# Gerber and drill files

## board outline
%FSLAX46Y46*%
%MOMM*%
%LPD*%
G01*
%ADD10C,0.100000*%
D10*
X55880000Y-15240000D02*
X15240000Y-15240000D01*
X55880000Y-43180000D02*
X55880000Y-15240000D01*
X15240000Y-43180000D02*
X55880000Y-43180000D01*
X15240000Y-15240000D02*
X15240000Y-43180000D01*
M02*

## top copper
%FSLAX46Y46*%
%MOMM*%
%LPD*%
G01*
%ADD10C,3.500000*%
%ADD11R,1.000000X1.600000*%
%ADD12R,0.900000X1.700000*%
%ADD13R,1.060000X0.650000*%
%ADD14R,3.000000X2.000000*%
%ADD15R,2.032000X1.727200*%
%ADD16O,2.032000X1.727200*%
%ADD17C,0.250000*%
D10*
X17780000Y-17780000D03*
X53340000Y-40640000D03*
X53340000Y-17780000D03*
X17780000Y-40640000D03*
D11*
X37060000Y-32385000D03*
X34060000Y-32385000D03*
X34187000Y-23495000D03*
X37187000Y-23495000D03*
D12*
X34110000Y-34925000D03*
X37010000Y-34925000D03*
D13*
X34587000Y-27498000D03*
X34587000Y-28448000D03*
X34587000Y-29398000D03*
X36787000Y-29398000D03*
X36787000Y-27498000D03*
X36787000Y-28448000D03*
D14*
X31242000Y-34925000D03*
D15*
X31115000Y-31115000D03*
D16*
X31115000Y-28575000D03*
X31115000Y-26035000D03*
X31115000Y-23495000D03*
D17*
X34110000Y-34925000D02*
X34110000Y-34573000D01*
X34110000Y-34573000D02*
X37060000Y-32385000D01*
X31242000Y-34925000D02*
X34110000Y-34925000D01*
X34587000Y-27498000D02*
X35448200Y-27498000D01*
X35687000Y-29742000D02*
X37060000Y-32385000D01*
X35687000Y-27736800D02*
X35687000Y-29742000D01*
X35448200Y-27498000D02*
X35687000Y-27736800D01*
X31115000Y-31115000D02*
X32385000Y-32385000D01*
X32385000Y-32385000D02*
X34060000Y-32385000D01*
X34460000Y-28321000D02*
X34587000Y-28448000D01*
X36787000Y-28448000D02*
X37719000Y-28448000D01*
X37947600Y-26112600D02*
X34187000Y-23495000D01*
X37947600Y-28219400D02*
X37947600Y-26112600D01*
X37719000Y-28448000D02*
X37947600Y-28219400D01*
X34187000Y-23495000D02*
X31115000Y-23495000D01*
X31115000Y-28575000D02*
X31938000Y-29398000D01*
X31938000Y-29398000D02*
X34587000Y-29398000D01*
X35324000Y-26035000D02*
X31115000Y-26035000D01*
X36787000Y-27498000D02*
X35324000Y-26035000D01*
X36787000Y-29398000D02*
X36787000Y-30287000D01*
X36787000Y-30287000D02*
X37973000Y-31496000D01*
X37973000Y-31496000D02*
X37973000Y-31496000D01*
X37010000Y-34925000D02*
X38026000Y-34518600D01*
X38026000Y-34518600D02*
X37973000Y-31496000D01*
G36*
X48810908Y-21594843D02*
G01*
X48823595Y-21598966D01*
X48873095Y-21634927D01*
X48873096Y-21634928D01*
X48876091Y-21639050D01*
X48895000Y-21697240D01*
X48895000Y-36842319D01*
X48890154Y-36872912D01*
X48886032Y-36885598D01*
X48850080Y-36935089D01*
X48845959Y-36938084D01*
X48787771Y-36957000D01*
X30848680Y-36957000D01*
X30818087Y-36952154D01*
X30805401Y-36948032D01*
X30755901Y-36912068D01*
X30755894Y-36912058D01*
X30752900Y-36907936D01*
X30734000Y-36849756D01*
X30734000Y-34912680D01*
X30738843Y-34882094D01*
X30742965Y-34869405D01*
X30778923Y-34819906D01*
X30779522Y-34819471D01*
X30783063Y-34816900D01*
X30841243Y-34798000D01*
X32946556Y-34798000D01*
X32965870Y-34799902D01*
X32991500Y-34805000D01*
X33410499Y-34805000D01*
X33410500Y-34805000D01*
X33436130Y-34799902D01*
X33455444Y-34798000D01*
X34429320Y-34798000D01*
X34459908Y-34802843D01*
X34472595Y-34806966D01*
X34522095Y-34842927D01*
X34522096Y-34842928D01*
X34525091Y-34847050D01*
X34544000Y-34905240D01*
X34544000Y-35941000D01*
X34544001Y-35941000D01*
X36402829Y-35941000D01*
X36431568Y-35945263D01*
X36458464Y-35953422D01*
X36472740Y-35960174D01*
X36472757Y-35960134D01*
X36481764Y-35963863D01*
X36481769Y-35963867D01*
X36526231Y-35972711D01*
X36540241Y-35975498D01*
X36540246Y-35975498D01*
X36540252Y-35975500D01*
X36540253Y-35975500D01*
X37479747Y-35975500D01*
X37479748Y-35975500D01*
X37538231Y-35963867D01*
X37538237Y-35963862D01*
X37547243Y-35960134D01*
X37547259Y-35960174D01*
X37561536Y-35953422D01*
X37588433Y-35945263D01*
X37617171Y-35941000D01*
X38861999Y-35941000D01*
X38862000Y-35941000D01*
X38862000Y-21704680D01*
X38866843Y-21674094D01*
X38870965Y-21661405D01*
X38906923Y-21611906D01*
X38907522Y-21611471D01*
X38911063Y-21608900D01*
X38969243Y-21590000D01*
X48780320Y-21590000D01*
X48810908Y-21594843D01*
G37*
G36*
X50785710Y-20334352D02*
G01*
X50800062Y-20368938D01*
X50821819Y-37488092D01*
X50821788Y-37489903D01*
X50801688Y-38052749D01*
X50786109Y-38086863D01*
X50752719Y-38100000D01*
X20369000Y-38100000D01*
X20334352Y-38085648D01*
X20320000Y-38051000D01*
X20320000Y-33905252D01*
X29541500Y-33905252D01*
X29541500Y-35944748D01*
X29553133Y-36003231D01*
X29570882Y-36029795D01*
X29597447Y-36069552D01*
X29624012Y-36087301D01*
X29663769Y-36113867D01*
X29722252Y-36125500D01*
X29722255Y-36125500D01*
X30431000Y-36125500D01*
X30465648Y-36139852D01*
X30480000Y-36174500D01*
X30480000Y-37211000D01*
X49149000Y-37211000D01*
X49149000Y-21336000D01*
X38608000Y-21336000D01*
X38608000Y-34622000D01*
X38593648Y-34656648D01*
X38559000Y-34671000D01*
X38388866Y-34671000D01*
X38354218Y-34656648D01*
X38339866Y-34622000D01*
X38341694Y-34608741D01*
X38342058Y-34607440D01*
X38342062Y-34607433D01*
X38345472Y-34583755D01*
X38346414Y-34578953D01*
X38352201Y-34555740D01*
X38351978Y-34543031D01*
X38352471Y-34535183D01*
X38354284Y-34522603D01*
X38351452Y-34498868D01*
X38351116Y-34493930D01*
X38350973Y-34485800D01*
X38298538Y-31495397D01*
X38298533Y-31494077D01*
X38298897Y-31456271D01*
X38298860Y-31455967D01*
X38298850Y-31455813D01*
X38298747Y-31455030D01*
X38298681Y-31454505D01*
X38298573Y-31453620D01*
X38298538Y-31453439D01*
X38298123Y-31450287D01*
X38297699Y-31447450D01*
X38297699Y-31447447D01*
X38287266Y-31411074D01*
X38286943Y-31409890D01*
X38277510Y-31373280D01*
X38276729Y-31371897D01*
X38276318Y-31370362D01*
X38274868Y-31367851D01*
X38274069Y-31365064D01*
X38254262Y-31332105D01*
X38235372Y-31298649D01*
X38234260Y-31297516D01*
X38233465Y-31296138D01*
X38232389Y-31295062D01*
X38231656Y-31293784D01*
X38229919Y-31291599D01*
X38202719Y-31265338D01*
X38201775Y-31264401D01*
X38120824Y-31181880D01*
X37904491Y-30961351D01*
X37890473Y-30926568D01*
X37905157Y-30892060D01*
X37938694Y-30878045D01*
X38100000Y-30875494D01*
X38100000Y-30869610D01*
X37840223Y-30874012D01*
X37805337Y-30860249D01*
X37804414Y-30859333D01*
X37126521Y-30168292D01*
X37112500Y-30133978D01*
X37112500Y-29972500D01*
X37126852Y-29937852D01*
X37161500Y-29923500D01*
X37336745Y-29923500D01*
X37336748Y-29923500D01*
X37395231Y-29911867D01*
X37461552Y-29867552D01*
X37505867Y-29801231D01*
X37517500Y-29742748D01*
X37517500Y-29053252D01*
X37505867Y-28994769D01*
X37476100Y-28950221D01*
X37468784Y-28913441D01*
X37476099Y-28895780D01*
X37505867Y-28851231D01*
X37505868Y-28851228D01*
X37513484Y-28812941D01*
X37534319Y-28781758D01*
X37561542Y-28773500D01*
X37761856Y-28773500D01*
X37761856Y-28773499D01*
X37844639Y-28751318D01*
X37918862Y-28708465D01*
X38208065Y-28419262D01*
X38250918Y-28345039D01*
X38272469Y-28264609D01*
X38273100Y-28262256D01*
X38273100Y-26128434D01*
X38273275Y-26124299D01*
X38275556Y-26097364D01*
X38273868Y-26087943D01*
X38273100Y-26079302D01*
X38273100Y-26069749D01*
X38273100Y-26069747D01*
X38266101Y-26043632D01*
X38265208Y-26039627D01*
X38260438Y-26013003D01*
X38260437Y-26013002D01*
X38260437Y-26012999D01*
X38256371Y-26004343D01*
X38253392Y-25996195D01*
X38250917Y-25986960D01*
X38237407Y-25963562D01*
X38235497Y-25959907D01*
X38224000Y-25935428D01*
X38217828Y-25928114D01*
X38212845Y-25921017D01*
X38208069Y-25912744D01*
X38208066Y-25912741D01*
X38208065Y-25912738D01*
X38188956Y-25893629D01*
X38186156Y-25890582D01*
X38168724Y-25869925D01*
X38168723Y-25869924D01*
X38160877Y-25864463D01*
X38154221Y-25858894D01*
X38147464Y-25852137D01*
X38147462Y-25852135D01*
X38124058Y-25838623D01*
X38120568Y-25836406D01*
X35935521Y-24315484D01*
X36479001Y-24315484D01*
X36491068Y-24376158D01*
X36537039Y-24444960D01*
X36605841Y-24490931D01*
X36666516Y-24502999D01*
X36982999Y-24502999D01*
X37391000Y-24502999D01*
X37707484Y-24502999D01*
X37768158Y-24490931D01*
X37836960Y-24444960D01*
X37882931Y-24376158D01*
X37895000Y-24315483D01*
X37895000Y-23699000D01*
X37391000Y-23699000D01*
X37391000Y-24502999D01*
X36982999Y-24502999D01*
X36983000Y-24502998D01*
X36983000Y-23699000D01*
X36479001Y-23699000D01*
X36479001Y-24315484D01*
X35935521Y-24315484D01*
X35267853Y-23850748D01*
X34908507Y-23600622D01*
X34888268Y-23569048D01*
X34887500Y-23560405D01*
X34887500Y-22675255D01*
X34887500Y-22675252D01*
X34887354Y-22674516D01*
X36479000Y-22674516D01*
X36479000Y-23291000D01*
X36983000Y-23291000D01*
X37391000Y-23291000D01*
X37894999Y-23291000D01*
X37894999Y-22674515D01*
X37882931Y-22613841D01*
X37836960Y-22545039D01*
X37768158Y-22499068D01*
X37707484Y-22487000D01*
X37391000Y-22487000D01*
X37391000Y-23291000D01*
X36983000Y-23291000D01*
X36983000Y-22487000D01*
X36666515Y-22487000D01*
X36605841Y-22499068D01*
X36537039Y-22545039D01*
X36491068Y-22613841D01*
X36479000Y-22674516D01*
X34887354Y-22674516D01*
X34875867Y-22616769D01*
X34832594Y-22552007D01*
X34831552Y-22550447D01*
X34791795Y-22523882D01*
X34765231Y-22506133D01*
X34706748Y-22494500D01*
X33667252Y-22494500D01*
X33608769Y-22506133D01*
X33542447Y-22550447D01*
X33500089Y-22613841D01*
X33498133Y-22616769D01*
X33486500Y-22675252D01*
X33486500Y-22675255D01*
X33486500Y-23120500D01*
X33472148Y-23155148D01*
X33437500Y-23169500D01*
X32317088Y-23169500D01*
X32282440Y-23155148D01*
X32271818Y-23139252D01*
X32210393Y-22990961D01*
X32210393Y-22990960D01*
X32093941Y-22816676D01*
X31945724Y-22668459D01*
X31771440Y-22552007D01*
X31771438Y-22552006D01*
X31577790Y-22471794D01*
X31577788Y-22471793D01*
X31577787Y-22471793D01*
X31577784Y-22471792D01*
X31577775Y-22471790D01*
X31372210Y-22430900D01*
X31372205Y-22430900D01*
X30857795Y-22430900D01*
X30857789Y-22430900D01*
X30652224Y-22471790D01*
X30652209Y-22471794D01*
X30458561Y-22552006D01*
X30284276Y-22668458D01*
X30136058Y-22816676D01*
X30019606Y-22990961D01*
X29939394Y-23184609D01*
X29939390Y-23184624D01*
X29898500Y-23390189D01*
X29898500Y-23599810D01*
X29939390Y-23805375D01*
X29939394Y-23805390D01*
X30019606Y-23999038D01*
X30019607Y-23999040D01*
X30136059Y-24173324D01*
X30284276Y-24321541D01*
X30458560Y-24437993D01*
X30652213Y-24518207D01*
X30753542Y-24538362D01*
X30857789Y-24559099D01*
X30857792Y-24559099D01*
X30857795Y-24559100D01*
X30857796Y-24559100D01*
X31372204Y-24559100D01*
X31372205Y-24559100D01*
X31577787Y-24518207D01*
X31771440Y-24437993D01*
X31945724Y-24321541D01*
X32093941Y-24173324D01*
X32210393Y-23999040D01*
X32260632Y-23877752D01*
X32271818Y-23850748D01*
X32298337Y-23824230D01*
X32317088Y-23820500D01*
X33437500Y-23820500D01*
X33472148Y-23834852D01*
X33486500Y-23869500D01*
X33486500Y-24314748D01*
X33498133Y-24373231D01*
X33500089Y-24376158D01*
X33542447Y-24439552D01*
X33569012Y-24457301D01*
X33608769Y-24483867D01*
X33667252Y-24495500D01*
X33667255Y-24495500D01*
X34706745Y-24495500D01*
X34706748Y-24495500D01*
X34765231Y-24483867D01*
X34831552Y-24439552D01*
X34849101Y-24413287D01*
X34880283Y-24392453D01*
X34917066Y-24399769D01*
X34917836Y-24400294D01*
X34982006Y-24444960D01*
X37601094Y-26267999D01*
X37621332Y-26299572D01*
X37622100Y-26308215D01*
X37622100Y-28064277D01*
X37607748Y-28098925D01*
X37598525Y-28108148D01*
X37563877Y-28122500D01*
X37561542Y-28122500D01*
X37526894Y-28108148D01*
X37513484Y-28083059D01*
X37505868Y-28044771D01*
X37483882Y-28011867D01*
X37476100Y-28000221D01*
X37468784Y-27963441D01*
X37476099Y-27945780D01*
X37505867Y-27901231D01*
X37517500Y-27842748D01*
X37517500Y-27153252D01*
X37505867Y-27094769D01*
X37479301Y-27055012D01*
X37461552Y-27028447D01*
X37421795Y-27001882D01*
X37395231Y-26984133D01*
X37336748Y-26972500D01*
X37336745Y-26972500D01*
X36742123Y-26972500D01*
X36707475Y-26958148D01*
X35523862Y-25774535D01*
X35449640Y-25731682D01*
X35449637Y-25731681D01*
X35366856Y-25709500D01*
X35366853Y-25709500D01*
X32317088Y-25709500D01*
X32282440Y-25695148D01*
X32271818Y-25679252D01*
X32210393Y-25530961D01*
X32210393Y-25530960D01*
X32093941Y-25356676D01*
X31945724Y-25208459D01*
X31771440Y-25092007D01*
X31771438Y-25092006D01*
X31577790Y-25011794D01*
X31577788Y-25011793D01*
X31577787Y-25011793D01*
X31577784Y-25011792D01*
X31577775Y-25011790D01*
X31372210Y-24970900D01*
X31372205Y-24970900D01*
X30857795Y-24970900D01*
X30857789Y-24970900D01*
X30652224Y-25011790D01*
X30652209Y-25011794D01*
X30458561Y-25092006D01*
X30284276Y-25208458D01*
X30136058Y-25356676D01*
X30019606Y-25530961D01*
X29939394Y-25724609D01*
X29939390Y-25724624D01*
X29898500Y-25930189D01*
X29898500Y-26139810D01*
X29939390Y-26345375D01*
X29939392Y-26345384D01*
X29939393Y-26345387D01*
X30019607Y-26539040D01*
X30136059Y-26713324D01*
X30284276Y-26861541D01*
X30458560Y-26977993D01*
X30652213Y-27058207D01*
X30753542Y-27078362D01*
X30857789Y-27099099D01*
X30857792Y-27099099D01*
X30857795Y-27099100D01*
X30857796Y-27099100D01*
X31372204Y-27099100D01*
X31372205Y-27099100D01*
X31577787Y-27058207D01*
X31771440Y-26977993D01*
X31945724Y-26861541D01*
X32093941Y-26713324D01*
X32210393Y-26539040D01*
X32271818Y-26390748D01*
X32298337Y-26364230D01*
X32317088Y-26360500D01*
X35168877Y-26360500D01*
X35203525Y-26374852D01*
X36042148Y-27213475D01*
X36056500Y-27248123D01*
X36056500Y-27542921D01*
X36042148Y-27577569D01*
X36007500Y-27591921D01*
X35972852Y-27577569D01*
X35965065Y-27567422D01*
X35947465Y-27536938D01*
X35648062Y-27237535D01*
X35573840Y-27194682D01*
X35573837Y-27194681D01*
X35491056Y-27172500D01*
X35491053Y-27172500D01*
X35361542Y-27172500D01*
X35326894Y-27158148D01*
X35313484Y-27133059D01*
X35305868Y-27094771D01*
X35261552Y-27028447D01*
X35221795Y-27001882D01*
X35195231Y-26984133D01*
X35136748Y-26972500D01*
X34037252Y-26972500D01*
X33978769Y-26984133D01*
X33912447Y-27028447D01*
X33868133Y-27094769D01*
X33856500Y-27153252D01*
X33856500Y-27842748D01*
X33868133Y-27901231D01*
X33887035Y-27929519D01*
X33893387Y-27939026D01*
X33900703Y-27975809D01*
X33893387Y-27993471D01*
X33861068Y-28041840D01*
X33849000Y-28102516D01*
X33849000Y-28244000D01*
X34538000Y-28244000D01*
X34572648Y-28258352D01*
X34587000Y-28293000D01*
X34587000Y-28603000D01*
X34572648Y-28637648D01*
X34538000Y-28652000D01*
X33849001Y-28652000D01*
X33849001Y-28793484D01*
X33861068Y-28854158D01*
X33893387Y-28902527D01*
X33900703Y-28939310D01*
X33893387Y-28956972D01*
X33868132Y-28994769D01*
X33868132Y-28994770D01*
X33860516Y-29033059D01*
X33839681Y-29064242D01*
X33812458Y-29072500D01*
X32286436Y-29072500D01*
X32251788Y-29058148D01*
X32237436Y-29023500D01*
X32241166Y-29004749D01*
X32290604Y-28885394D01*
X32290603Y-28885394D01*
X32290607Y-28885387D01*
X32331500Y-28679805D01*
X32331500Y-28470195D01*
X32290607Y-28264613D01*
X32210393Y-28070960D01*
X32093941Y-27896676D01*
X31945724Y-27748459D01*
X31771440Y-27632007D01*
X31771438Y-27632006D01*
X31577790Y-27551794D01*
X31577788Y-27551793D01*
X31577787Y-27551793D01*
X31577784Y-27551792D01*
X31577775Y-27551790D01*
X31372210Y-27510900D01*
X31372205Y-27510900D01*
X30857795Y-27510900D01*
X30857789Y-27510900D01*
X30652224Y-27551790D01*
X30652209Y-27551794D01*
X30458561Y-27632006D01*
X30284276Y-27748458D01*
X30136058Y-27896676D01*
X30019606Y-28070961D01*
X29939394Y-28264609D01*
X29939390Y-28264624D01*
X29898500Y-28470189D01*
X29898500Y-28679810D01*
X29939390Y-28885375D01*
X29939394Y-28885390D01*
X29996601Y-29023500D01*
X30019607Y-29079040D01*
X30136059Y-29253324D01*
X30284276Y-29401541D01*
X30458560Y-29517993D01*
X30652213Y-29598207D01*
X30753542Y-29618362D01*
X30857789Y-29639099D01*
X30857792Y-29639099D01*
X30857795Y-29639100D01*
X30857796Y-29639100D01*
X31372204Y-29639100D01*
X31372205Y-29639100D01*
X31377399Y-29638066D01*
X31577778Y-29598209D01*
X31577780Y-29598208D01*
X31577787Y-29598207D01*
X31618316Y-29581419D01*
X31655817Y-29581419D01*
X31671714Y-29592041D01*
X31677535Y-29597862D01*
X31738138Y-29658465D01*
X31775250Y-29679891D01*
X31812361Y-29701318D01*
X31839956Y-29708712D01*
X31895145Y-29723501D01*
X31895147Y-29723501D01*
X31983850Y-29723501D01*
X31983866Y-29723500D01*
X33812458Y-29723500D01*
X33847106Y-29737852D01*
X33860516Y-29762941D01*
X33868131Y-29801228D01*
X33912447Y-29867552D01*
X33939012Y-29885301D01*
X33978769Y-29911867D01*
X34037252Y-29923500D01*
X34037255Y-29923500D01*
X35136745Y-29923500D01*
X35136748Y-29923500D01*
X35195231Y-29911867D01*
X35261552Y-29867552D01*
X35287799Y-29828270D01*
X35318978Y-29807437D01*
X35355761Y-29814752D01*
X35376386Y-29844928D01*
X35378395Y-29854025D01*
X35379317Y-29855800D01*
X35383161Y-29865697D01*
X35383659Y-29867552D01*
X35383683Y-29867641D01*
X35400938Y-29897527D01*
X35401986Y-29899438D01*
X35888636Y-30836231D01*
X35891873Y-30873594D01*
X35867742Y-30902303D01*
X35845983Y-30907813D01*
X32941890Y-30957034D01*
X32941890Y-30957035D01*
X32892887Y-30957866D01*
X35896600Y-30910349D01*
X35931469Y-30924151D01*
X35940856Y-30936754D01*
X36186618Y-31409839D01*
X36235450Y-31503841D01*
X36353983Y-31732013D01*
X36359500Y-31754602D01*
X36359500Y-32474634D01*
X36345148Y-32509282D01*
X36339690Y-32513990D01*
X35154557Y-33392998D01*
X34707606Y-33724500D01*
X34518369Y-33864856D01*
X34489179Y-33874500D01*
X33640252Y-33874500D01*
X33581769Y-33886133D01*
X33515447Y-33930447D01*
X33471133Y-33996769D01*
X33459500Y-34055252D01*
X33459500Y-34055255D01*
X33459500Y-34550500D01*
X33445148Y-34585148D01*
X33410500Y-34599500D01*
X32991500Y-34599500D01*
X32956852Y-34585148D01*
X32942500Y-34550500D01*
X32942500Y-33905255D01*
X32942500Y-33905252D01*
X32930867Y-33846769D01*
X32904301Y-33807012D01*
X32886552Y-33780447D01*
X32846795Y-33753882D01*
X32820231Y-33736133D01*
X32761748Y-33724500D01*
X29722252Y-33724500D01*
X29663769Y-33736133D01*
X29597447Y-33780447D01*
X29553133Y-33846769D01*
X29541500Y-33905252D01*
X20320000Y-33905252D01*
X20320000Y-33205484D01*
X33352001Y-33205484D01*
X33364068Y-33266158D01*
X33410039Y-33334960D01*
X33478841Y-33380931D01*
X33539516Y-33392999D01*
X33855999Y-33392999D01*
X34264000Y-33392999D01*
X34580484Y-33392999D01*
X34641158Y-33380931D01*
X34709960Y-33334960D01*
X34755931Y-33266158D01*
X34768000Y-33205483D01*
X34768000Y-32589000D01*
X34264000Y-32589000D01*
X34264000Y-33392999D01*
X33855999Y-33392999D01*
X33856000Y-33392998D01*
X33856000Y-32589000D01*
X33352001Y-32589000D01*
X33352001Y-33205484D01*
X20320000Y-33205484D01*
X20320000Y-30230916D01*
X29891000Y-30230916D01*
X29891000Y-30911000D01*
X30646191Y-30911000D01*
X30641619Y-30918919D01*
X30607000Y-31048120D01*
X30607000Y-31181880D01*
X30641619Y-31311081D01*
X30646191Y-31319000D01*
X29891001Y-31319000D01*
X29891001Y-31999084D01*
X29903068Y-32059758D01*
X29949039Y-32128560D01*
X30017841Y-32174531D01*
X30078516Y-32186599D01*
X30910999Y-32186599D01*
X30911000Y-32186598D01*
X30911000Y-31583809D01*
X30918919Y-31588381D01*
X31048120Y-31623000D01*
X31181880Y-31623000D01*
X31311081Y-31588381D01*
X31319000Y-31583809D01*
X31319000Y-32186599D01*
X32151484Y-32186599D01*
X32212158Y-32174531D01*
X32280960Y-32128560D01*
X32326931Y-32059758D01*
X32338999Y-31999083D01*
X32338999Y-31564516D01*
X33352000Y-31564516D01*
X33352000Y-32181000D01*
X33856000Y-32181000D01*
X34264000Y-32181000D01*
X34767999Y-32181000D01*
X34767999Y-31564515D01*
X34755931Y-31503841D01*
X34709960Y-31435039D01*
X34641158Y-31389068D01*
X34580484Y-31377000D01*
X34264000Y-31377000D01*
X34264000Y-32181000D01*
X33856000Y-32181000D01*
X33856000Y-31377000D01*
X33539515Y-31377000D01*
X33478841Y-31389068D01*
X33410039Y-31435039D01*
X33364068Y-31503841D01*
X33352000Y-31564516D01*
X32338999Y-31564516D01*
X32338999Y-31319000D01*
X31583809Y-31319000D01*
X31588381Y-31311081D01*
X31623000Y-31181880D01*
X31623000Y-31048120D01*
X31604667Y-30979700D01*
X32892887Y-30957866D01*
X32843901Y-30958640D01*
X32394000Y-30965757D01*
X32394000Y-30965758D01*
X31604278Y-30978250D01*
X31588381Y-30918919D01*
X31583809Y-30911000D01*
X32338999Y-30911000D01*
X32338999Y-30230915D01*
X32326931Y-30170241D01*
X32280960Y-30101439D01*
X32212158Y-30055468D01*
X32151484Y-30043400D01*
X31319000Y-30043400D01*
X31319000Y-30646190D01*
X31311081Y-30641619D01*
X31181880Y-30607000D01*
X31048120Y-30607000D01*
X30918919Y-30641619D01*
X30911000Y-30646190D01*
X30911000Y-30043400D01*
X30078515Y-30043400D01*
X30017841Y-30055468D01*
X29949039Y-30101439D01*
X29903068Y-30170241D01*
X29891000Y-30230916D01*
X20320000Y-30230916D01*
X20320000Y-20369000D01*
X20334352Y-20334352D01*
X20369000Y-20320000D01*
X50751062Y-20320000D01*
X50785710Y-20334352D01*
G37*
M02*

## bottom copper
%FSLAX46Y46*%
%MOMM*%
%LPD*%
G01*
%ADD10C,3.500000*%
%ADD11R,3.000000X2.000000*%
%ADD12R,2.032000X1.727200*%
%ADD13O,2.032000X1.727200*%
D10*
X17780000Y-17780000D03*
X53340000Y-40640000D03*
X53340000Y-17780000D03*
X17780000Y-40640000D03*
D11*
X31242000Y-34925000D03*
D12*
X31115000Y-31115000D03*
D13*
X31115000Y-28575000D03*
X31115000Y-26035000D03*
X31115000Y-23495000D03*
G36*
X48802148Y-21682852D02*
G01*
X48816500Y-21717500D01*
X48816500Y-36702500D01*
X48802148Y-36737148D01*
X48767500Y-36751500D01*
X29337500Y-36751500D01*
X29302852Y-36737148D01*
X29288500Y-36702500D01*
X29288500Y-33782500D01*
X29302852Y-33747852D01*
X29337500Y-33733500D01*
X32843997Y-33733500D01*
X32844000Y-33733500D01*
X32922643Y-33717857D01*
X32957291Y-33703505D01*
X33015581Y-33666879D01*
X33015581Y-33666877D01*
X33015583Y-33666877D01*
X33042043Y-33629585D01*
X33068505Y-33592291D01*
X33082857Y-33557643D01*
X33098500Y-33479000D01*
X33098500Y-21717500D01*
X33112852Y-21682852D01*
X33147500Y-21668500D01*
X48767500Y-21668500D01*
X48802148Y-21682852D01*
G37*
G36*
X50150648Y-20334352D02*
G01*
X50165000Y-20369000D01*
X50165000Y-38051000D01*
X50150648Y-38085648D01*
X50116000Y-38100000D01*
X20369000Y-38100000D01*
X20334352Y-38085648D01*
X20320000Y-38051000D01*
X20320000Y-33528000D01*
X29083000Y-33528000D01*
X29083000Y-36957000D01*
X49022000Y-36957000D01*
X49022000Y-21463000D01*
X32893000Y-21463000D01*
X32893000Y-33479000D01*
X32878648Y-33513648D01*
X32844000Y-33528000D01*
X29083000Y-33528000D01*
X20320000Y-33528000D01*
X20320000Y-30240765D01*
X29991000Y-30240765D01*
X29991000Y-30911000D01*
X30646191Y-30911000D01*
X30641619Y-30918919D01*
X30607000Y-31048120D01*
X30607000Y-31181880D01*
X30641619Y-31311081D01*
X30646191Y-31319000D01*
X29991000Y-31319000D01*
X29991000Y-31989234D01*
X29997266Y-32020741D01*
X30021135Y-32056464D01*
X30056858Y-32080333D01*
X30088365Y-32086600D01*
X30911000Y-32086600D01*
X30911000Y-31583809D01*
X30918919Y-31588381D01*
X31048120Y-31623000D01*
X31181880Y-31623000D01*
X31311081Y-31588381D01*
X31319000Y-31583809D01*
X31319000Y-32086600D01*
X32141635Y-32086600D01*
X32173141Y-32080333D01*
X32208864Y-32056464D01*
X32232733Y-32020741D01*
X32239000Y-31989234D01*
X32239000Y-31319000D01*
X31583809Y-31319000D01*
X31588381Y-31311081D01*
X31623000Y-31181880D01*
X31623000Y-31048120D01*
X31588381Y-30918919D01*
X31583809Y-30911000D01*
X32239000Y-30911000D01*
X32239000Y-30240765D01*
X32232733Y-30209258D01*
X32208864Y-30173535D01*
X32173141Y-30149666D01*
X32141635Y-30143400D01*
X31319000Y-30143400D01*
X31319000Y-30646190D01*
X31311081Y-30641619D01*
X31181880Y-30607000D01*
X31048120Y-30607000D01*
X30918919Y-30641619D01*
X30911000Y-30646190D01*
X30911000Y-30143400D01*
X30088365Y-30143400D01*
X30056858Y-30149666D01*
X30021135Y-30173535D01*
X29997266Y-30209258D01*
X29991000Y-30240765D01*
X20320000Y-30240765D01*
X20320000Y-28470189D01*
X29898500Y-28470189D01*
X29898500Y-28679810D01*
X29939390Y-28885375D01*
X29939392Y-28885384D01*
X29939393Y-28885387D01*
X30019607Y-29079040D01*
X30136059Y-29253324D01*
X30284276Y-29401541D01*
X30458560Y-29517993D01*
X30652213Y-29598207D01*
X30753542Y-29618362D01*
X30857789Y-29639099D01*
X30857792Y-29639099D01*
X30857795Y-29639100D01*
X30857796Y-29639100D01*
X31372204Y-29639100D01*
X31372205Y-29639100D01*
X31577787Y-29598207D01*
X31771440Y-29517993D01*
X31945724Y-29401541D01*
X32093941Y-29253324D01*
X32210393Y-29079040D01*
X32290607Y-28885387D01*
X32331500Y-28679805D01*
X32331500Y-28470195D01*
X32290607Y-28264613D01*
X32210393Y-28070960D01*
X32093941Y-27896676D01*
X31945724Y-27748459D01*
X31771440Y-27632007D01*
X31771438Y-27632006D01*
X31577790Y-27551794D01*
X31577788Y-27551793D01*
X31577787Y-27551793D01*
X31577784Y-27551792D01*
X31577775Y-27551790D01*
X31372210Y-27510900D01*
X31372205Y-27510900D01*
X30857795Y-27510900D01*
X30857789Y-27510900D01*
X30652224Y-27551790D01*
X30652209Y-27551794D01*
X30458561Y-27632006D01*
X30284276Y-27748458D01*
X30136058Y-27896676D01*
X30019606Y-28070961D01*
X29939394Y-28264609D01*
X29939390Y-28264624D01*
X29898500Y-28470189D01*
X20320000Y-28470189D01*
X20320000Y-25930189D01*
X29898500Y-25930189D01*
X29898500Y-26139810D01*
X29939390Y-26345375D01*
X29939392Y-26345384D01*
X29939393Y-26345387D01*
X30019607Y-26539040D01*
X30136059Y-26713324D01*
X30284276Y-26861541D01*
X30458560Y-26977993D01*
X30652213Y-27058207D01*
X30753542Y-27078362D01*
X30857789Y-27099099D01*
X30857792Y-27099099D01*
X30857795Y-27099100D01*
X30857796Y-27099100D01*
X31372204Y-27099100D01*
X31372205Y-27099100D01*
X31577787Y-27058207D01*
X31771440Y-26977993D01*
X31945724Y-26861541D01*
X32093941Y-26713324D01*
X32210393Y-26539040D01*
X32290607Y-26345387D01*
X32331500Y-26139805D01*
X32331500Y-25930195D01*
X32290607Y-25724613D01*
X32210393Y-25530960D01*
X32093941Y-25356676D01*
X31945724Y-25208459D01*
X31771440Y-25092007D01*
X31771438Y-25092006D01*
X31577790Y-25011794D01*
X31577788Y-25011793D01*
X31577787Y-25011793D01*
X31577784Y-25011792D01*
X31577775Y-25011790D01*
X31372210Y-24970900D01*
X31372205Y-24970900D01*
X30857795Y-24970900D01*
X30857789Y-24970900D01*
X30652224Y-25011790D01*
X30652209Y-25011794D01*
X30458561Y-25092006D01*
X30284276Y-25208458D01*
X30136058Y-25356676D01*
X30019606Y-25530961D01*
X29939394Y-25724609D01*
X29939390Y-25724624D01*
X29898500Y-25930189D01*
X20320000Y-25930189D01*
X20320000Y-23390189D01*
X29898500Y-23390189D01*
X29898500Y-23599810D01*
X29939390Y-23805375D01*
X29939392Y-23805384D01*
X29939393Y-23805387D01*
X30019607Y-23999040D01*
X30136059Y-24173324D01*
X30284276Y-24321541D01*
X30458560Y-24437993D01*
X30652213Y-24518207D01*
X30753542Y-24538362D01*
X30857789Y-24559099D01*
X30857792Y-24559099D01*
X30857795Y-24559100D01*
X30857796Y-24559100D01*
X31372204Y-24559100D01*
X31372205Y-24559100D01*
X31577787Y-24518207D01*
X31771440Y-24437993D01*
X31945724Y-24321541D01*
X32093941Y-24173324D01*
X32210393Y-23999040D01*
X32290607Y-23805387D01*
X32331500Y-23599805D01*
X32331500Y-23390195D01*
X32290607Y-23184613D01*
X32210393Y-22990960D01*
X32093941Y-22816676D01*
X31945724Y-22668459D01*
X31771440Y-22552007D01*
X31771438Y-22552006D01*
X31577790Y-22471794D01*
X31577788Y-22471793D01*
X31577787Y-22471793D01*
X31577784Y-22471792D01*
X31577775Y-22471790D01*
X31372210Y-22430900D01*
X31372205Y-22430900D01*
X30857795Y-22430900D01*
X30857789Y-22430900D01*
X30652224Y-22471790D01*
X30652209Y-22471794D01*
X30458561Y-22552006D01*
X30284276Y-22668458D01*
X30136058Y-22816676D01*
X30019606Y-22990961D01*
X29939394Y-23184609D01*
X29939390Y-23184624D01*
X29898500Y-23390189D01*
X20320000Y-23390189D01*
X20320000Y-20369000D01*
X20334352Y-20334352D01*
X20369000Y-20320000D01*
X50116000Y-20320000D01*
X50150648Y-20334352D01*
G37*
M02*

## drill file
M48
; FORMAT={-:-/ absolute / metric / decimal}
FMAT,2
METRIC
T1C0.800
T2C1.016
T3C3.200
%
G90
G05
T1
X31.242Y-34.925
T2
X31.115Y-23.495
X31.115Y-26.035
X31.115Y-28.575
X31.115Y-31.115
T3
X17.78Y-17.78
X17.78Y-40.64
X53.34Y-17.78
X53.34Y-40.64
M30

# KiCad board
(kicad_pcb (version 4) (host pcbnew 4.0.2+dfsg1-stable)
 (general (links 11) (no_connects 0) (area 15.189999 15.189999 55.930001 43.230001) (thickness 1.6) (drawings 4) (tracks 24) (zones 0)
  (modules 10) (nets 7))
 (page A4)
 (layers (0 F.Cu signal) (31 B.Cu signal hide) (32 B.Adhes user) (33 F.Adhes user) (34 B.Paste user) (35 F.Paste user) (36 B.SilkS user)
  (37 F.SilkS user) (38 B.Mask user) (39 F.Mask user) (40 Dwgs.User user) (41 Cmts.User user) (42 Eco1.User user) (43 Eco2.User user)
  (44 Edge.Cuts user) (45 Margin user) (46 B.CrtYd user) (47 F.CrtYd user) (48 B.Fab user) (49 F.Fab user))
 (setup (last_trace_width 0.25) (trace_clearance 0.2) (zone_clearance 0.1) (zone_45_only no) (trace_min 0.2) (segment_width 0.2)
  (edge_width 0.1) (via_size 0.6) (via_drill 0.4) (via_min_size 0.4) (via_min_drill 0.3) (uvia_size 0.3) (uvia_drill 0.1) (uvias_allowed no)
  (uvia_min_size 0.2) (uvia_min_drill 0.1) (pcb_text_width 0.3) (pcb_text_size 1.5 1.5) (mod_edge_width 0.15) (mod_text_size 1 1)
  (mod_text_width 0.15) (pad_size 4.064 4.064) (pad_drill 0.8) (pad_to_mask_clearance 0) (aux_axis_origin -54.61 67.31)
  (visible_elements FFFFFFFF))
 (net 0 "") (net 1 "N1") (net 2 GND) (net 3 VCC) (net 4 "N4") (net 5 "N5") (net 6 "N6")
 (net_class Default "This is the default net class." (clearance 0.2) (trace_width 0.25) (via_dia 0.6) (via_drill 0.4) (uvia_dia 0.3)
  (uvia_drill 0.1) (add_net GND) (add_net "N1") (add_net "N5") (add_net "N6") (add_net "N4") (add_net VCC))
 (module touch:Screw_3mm (layer F.Cu) (at 17.78 17.78)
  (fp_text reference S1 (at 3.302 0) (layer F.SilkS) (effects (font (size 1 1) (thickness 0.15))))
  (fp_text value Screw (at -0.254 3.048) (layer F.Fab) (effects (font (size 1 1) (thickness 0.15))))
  (pad 1 thru_hole circle (at 0 0) (size 3.5 3.5) (drill 3.2) (layers *.Cu *.Mask F.SilkS)))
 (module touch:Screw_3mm (layer F.Cu) (at 53.34 40.64)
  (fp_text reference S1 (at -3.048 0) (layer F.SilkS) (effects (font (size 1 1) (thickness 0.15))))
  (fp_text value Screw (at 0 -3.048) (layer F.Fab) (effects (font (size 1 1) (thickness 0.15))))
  (pad 1 thru_hole circle (at 0 0) (size 3.5 3.5) (drill 3.2) (layers *.Cu *.Mask F.SilkS)))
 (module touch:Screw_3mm (layer F.Cu) (at 53.34 17.78)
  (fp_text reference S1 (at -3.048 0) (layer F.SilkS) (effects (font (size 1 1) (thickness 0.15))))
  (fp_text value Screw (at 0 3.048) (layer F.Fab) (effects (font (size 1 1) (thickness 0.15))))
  (pad 1 thru_hole circle (at 0 0) (size 3.5 3.5) (drill 3.2) (layers *.Cu *.Mask F.SilkS)))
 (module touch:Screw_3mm (layer F.Cu) (at 17.78 40.64)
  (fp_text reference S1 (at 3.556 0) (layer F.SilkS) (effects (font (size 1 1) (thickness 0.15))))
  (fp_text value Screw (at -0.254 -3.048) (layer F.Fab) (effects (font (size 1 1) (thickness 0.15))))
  (pad 1 thru_hole circle (at 0 0) (size 3.5 3.5) (drill 3.2) (layers *.Cu *.Mask F.SilkS)))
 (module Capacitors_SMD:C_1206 (layer F.Cu) (at 35.56 32.385 180)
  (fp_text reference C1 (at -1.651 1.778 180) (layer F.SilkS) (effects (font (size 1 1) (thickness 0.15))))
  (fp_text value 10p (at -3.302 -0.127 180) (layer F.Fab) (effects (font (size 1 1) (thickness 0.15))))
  (pad 1 smd rect (at -1.5 0 180) (size 1 1.6) (layers F.Cu F.Paste F.Mask) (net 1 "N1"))
  (pad 2 smd rect (at 1.5 0 180) (size 1 1.6) (layers F.Cu F.Paste F.Mask) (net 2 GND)))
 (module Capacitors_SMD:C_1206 (layer F.Cu) (at 35.687 23.495)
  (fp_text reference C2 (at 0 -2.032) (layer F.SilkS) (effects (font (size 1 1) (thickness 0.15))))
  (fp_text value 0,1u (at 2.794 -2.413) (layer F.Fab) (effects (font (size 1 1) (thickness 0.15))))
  (pad 1 smd rect (at -1.5 0) (size 1 1.6) (layers F.Cu F.Paste F.Mask) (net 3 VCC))
  (pad 2 smd rect (at 1.5 0) (size 1 1.6) (layers F.Cu F.Paste F.Mask) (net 2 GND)))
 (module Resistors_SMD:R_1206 (layer F.Cu) (at 35.56 34.925)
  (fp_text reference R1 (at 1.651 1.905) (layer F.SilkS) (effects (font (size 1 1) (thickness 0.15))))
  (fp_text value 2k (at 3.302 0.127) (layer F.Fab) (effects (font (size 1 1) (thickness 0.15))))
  (pad 1 smd rect (at -1.45 0) (size 0.9 1.7) (layers F.Cu F.Paste F.Mask) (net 1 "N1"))
  (pad 2 smd rect (at 1.45 0) (size 0.9 1.7) (layers F.Cu F.Paste F.Mask) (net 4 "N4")))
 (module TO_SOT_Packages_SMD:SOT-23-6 (layer F.Cu) (at 35.687 28.448)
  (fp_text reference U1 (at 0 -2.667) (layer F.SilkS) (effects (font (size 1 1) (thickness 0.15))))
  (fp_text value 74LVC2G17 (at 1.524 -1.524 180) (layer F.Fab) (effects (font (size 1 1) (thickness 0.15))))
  (pad 1 smd rect (at -1.1 -0.95) (size 1.06 0.65) (layers F.Cu F.Paste F.Mask) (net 1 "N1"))
  (pad 2 smd rect (at -1.1 0) (size 1.06 0.65) (layers F.Cu F.Paste F.Mask) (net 2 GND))
  (pad 3 smd rect (at -1.1 0.95) (size 1.06 0.65) (layers F.Cu F.Paste F.Mask) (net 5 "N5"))
  (pad 4 smd rect (at 1.1 0.95) (size 1.06 0.65) (layers F.Cu F.Paste F.Mask) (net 4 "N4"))
  (pad 6 smd rect (at 1.1 -0.95) (size 1.06 0.65) (layers F.Cu F.Paste F.Mask) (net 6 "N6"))
  (pad 5 smd rect (at 1.1 0) (size 1.06 0.65) (layers F.Cu F.Paste F.Mask) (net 3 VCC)))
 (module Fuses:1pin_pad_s (layer F.Cu) (at 31.242 34.925)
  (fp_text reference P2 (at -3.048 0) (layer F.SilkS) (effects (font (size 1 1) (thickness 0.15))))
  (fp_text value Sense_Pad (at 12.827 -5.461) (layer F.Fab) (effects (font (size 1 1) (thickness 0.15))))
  (pad 1 thru_hole rect (at 0 0) (size 3 2) (drill 0.8) (layers *.Cu *.Mask F.SilkS) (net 1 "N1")))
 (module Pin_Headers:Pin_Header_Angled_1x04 (layer F.Cu) (at 31.115 31.115 180)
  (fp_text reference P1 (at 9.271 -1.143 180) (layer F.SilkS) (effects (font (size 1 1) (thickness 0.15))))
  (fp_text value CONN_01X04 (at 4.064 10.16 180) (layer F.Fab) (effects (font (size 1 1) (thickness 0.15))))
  (pad 1 thru_hole rect (at 0 0 180) (size 2.032 1.7272) (drill 1.016) (layers *.Cu *.Mask F.SilkS) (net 2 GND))
  (pad 2 thru_hole oval (at 0 2.54 180) (size 2.032 1.7272) (drill 1.016) (layers *.Cu *.Mask F.SilkS) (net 5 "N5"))
  (pad 3 thru_hole oval (at 0 5.08 180) (size 2.032 1.7272) (drill 1.016) (layers *.Cu *.Mask F.SilkS) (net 6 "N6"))
  (pad 4 thru_hole oval (at 0 7.62 180) (size 2.032 1.7272) (drill 1.016) (layers *.Cu *.Mask F.SilkS) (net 3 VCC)))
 (gr_line (start 55.88 15.24) (end 15.24 15.24) (angle 90) (layer Edge.Cuts) (width 0.1))
 (gr_line (start 55.88 43.18) (end 55.88 15.24) (angle 90) (layer Edge.Cuts) (width 0.1))
 (gr_line (start 15.24 43.18) (end 55.88 43.18) (angle 90) (layer Edge.Cuts) (width 0.1))
 (gr_line (start 15.24 15.24) (end 15.24 43.18) (angle 90) (layer Edge.Cuts) (width 0.1))
 (segment (start 34.11 34.925) (end 34.11 34.573) (width 0.25) (layer F.Cu) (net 1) (status 30))
 (segment (start 34.11 34.573) (end 37.06 32.385) (width 0.25) (layer F.Cu) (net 1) (status 20))
 (segment (start 31.242 34.925) (end 34.11 34.925) (width 0.25) (layer F.Cu) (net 1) (status 10))
 (segment (start 34.587 27.498) (end 35.4482 27.498) (width 0.25) (layer F.Cu) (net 1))
 (segment (start 35.687 29.742) (end 37.06 32.385) (width 0.25) (layer F.Cu) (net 1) (status 20))
 (segment (start 35.687 27.7368) (end 35.687 29.742) (width 0.25) (layer F.Cu) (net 1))
 (segment (start 35.4482 27.498) (end 35.687 27.7368) (width 0.25) (layer F.Cu) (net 1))
 (segment (start 31.115 31.115) (end 32.385 32.385) (width 0.25) (layer F.Cu) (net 2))
 (segment (start 32.385 32.385) (end 34.06 32.385) (width 0.25) (layer F.Cu) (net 2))
 (segment (start 34.46 28.321) (end 34.587 28.448) (width 0.25) (layer F.Cu) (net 2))
 (segment (start 36.787 28.448) (end 37.719 28.448) (width 0.25) (layer F.Cu) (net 3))
 (segment (start 37.9476 26.1126) (end 34.187 23.495) (width 0.25) (layer F.Cu) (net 3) (status 20))
 (segment (start 37.9476 28.2194) (end 37.9476 26.1126) (width 0.25) (layer F.Cu) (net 3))
 (segment (start 37.719 28.448) (end 37.9476 28.2194) (width 0.25) (layer F.Cu) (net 3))
 (segment (start 34.187 23.495) (end 31.115 23.495) (width 0.25) (layer F.Cu) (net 3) (status 10))
 (segment (start 31.115 28.575) (end 31.938 29.398) (width 0.25) (layer F.Cu) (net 5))
 (segment (start 31.938 29.398) (end 34.587 29.398) (width 0.25) (layer F.Cu) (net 5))
 (segment (start 35.324 26.035) (end 31.115 26.035) (width 0.25) (layer F.Cu) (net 6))
 (segment (start 36.787 27.498) (end 35.324 26.035) (width 0.25) (layer F.Cu) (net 6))
 (segment (start 36.787 29.398) (end 36.787 30.287) (width 0.25) (layer F.Cu) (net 4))
 (segment (start 36.787 30.287) (end 37.973 31.496) (width 0.25) (layer F.Cu) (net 4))
 (segment (start 37.973 31.496) (end 37.973 31.496) (width 0.25) (layer F.Cu) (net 4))
 (segment (start 37.01 34.925) (end 38.026 34.5186) (width 0.25) (layer F.Cu) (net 4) (status 10))
 (segment (start 38.026 34.5186) (end 37.973 31.496) (width 0.25) (layer F.Cu) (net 4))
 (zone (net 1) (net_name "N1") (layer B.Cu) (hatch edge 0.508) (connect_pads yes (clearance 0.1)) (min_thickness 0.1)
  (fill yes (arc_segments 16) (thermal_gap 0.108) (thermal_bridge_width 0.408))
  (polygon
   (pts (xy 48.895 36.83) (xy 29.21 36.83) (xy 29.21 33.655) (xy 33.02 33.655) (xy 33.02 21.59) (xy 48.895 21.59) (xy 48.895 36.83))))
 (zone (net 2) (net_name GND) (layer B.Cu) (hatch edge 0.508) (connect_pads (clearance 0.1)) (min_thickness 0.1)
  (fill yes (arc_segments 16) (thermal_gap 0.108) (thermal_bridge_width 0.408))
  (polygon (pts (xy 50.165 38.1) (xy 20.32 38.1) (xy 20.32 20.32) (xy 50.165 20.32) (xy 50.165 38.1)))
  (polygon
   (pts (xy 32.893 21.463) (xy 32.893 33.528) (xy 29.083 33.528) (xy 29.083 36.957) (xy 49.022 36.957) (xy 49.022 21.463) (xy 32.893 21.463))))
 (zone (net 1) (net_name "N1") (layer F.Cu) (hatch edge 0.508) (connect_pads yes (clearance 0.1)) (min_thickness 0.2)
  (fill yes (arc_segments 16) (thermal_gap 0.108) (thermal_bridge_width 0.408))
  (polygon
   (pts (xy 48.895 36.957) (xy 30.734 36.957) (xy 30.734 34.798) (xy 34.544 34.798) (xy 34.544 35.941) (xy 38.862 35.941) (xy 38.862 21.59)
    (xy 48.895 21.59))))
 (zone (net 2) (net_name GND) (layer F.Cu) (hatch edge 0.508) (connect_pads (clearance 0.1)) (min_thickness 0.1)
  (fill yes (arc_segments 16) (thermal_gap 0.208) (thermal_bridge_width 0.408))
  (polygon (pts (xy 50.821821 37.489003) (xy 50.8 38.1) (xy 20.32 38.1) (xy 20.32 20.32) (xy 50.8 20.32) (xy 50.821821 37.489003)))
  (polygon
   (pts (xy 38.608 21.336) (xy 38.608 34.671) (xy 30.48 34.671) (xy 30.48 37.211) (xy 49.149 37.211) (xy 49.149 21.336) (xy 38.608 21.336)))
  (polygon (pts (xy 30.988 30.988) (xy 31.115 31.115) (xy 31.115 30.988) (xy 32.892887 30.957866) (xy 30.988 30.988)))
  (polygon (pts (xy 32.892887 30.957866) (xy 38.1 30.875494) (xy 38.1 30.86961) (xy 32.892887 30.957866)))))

